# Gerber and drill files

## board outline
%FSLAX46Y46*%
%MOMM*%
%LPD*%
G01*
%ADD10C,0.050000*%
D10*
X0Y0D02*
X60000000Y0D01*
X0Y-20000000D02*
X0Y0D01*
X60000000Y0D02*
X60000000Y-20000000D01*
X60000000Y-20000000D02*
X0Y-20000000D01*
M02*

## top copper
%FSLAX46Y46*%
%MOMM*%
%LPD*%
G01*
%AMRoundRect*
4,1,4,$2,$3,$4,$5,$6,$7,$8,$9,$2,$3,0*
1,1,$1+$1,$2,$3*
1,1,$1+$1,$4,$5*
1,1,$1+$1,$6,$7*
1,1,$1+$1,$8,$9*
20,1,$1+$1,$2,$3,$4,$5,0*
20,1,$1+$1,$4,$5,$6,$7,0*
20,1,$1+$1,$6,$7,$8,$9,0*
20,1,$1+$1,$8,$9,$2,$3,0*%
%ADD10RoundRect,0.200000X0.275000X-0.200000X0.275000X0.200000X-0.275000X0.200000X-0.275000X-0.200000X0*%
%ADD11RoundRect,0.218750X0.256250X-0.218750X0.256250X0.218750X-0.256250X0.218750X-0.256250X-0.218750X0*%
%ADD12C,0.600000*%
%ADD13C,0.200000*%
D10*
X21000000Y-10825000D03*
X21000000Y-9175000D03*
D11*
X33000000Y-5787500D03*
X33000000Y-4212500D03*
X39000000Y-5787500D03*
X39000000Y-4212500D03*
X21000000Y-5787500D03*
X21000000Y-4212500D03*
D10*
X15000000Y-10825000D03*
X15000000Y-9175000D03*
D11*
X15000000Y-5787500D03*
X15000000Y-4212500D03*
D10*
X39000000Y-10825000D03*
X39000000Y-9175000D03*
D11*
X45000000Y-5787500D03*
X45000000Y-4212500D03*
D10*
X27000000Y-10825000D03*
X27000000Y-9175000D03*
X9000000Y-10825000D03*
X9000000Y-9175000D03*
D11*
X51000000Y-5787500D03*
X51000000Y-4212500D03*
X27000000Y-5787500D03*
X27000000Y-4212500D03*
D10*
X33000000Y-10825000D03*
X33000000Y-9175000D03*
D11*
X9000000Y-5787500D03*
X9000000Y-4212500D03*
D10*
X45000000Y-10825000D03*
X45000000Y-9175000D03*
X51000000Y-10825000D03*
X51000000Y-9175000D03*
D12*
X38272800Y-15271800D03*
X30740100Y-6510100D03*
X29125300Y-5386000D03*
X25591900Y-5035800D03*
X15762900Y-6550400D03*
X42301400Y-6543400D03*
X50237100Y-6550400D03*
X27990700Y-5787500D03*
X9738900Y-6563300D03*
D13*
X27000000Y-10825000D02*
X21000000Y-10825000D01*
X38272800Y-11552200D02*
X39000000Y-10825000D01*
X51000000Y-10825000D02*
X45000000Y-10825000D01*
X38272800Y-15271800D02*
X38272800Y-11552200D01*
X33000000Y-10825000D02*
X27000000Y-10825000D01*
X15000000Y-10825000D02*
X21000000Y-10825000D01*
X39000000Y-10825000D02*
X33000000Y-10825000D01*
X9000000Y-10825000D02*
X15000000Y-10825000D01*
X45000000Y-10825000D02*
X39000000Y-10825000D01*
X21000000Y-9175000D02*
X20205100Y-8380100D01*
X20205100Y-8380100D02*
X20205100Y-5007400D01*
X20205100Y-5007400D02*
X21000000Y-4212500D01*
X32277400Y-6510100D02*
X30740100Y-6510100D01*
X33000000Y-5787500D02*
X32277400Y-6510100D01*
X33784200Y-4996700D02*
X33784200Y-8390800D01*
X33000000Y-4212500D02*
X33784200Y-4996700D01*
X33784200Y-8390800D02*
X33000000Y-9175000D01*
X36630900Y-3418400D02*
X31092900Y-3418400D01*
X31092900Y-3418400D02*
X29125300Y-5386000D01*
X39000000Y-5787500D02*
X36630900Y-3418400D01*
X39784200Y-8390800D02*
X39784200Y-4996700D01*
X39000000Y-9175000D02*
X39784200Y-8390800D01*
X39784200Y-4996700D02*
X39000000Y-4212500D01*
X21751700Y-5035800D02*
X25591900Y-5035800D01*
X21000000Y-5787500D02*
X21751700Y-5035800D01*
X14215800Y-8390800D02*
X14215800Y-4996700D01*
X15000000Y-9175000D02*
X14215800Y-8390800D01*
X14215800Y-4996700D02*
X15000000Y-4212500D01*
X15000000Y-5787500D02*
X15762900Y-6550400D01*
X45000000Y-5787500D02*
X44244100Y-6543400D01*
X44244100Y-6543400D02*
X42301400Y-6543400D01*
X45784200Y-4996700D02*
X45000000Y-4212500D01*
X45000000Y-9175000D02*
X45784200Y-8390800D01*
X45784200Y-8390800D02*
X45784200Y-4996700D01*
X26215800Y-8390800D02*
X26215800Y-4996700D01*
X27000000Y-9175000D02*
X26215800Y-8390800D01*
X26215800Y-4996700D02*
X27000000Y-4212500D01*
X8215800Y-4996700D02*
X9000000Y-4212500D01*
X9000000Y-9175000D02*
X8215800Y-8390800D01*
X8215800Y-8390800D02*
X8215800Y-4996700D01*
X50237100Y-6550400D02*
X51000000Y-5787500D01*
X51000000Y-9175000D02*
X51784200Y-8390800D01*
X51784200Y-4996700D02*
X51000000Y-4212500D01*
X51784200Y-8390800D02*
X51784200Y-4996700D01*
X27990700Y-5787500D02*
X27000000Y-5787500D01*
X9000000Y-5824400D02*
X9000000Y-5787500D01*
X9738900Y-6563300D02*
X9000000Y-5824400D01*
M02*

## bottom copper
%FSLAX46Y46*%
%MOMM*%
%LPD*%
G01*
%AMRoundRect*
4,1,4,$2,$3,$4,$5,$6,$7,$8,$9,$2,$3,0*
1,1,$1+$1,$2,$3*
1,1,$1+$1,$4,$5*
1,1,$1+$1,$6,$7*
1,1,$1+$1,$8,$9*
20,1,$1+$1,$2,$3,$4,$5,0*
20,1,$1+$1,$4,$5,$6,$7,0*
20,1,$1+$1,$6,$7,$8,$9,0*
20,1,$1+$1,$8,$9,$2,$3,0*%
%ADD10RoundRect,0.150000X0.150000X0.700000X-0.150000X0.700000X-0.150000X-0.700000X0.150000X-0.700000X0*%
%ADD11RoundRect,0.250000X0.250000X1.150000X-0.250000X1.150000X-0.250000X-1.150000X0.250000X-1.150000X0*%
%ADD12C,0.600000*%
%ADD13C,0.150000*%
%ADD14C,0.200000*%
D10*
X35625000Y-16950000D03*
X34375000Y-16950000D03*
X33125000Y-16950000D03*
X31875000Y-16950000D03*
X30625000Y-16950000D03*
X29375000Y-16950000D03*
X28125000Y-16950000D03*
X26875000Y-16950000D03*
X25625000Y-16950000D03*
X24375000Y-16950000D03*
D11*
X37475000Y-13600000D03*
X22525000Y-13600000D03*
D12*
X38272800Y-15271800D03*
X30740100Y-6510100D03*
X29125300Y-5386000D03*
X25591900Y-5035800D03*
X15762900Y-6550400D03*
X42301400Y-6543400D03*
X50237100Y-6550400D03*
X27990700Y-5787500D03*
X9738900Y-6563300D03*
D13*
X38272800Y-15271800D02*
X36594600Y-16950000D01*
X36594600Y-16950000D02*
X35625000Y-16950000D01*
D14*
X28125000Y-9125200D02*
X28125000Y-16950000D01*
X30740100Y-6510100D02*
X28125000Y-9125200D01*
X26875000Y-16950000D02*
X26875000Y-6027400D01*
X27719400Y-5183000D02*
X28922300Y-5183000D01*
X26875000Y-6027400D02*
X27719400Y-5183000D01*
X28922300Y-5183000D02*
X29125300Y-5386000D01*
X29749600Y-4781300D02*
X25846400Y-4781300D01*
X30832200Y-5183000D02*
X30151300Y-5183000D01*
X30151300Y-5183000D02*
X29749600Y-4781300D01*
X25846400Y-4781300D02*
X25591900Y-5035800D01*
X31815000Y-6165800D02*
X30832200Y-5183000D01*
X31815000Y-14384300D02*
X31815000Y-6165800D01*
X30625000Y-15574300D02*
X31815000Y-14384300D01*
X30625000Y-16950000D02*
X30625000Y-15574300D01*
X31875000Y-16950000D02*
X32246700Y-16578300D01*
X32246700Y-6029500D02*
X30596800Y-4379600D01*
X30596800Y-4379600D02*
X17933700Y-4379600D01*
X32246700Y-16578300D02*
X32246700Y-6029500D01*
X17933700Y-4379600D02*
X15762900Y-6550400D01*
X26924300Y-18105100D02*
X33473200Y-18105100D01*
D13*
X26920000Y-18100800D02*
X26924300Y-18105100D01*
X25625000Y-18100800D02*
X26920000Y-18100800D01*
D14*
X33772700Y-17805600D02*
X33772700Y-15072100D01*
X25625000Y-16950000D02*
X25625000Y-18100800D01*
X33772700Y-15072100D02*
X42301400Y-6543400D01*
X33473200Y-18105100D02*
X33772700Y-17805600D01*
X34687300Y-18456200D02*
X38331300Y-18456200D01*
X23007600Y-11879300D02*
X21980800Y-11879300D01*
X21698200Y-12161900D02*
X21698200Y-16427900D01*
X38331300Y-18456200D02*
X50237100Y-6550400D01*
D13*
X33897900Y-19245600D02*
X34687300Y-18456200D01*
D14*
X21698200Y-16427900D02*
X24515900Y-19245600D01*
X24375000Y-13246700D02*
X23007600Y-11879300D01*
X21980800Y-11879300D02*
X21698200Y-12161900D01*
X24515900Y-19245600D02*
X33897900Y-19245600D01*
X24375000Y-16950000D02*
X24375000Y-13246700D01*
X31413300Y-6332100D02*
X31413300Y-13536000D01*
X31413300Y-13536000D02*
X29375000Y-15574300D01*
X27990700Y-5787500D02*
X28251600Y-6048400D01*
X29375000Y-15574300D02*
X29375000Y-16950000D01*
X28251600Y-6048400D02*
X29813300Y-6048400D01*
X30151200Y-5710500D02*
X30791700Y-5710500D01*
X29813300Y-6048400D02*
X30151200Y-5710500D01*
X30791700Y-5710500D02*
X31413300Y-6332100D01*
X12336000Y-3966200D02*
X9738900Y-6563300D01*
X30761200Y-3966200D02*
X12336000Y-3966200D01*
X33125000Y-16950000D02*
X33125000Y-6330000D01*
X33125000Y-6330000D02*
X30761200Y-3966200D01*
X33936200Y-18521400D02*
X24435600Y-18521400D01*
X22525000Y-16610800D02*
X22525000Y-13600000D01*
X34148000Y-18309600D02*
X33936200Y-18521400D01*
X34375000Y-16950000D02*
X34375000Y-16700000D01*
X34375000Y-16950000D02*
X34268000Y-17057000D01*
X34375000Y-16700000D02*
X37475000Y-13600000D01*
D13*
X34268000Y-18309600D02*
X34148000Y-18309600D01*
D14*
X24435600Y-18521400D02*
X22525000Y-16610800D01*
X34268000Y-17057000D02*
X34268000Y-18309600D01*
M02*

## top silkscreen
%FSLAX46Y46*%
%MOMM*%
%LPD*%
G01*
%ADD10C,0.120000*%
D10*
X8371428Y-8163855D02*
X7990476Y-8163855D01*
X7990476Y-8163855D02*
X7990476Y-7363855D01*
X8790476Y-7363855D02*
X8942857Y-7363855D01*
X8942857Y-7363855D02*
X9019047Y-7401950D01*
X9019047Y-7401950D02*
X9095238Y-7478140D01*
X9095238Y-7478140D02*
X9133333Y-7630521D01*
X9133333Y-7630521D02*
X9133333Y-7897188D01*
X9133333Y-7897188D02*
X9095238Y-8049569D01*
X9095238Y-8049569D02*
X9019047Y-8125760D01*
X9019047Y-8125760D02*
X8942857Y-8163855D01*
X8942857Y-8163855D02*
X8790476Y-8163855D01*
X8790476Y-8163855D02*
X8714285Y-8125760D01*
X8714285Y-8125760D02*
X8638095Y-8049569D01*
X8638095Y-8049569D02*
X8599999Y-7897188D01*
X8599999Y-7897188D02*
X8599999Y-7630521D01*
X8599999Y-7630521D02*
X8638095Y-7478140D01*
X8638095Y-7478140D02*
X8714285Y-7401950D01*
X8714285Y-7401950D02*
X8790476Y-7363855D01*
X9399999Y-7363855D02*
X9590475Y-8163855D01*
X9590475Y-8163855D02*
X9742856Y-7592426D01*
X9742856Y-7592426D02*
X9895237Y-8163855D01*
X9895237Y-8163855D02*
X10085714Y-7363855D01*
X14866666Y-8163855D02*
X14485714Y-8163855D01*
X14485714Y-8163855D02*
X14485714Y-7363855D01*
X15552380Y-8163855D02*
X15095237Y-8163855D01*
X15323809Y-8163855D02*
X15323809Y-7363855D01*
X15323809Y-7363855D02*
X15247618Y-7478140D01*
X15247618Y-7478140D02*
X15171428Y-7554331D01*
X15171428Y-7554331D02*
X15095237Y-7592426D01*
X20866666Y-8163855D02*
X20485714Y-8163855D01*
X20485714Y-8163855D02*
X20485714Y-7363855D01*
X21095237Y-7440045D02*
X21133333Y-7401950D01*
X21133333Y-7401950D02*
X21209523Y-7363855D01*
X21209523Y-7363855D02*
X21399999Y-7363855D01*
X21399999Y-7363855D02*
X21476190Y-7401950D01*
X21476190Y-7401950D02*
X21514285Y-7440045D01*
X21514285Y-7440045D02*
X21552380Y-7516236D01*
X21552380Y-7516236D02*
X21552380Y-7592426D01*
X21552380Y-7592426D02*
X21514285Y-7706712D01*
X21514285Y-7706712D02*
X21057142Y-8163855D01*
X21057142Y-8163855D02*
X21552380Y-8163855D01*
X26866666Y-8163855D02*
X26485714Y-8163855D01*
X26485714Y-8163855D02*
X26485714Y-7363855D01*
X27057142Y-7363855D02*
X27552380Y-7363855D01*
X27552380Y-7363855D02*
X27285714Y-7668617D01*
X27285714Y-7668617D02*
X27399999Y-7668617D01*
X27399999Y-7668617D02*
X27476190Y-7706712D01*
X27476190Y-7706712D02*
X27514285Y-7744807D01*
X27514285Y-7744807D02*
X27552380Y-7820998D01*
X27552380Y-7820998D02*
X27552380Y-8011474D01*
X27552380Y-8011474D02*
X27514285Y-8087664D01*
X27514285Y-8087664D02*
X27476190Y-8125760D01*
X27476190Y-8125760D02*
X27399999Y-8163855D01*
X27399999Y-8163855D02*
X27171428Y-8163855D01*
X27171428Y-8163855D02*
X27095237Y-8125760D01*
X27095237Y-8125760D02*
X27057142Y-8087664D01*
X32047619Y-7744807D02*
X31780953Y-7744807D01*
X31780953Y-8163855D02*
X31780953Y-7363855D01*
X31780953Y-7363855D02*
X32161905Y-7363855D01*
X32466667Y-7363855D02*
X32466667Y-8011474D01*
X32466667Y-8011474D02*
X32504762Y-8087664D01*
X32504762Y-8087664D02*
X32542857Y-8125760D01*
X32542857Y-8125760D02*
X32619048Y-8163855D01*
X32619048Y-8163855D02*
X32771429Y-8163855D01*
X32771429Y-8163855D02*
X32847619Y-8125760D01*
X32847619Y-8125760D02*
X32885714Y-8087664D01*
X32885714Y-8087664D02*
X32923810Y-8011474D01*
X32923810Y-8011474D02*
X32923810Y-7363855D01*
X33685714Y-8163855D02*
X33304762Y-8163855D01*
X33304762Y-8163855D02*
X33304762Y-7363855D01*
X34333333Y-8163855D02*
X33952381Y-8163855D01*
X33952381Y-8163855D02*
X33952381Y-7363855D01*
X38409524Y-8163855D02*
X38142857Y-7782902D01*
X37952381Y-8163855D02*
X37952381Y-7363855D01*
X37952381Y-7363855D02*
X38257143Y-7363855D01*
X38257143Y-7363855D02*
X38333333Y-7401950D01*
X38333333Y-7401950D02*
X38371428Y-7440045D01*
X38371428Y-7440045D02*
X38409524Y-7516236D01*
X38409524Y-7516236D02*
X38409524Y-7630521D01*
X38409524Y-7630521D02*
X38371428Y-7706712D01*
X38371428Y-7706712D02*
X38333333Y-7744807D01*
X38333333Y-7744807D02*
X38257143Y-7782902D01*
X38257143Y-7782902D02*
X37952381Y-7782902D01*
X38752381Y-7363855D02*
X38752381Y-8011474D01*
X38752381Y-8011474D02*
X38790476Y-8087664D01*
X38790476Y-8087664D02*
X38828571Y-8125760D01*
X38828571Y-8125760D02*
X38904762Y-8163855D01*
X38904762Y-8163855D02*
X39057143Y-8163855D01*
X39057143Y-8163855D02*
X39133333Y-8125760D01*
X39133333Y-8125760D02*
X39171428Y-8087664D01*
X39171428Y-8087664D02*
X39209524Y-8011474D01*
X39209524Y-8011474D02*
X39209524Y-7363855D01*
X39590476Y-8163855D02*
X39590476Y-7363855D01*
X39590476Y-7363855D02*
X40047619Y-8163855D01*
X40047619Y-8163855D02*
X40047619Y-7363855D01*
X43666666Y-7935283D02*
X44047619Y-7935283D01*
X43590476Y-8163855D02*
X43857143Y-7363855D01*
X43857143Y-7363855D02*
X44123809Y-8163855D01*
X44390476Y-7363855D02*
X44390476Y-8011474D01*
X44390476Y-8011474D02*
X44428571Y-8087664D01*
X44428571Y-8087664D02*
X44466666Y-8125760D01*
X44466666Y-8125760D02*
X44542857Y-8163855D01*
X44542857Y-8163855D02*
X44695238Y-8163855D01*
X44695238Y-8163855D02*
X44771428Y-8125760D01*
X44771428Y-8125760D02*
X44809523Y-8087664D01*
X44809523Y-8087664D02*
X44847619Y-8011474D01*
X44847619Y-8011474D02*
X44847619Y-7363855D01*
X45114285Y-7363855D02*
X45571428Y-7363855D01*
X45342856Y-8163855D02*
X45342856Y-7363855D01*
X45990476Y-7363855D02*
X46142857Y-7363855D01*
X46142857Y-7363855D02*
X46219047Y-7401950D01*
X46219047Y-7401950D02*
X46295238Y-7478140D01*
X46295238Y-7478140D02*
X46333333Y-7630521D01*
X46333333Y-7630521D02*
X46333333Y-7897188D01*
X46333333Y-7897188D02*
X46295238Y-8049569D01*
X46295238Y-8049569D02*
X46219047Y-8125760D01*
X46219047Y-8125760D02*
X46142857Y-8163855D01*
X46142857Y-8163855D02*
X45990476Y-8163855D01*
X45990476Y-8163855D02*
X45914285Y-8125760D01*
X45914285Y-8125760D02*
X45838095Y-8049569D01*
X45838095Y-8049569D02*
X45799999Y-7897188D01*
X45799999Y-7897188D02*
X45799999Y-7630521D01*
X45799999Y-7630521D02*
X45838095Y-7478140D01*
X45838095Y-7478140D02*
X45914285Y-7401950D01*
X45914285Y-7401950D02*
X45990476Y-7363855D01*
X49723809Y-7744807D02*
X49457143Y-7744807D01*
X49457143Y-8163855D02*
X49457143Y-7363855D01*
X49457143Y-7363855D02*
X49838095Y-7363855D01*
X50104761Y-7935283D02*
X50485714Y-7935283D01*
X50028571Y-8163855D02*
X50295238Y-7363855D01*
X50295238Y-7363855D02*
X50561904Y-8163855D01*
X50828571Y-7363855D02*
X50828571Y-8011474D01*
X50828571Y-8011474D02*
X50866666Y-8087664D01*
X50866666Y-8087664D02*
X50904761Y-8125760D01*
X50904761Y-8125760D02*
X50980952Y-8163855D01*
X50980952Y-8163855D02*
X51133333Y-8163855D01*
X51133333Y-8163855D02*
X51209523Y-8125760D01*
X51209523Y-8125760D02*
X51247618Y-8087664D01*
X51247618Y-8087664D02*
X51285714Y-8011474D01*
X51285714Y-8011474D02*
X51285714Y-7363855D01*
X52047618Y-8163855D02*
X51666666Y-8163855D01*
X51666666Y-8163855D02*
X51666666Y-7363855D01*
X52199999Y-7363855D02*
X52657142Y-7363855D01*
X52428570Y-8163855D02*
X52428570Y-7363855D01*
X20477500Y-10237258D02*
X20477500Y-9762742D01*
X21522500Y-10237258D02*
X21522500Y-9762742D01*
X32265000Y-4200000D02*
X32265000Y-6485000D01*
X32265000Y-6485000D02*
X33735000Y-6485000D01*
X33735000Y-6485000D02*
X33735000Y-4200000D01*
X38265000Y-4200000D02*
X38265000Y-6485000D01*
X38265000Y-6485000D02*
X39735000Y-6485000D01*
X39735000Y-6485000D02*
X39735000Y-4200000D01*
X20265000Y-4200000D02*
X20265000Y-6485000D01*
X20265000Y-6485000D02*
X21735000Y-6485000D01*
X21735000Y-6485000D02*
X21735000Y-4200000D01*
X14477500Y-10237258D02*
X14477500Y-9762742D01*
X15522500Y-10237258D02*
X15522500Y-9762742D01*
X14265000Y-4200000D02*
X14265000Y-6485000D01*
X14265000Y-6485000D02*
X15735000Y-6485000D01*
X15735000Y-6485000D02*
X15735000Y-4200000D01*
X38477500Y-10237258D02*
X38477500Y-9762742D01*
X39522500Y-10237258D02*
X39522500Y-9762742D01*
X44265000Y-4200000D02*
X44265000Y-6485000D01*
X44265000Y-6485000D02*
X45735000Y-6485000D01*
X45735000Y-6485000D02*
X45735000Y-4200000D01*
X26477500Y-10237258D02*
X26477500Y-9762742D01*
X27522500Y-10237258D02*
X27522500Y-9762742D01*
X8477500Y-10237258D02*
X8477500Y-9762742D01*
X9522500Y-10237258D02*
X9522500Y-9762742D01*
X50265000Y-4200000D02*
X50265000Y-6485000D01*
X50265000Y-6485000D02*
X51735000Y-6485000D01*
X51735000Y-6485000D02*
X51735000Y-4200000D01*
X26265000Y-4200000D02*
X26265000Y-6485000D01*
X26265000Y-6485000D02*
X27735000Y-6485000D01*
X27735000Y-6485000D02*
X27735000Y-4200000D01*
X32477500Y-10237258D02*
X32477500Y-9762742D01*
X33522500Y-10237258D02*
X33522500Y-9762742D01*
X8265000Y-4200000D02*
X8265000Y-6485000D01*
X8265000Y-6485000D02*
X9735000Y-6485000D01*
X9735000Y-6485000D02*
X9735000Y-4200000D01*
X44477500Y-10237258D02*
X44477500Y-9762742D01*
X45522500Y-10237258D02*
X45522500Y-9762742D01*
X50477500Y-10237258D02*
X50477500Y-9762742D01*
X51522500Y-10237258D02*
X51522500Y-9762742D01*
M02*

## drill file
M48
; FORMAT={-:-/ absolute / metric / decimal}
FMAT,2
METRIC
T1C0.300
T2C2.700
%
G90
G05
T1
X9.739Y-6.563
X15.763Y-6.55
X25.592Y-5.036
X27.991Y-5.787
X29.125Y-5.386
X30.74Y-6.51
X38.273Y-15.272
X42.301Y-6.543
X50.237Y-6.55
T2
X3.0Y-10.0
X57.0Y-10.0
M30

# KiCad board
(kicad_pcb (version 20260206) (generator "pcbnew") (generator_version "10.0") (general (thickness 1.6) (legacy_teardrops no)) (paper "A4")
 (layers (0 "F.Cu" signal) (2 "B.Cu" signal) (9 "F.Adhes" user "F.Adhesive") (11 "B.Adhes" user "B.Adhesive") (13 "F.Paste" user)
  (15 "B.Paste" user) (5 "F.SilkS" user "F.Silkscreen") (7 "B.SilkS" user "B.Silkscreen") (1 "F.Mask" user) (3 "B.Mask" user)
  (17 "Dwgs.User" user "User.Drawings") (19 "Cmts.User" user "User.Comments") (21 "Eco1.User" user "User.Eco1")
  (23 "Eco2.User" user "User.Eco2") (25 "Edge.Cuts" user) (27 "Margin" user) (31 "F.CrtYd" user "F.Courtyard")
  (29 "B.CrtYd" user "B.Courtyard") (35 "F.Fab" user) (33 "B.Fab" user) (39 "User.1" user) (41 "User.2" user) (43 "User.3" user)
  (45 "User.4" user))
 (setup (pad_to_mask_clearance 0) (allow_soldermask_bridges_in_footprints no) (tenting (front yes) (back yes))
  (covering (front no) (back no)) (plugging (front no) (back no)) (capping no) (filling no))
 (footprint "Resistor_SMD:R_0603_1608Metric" (layer "F.Cu") (at 21 10 90)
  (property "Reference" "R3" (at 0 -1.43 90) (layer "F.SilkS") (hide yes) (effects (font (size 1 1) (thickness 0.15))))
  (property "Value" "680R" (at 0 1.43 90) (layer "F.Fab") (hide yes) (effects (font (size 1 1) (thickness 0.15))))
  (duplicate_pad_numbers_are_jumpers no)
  (fp_line (start -0.237258 -0.5225) (end 0.237258 -0.5225) (stroke (width 0.12) (type solid)) (layer "F.SilkS"))
  (fp_line (start -0.237258 0.5225) (end 0.237258 0.5225) (stroke (width 0.12) (type solid)) (layer "F.SilkS"))
  (pad "1" smd roundrect (at -0.825 0 90) (size 0.8 0.95) (layers "F.Cu" "F.Mask" "F.Paste") (roundrect_rratio 0.25) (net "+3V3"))
  (pad "2" smd roundrect (at 0.825 0 90) (size 0.8 0.95) (layers "F.Cu" "F.Mask" "F.Paste") (roundrect_rratio 0.25) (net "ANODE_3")))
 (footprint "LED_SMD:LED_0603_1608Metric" (layer "F.Cu") (at 33 5 90)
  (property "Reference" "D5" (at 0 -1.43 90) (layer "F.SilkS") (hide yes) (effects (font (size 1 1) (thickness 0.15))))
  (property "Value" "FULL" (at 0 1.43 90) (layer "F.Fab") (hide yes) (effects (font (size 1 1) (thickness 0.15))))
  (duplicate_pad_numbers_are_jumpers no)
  (fp_line (start 0.8 -0.735) (end -1.485 -0.735) (stroke (width 0.12) (type solid)) (layer "F.SilkS"))
  (fp_line (start -1.485 -0.735) (end -1.485 0.735) (stroke (width 0.12) (type solid)) (layer "F.SilkS"))
  (fp_line (start -1.485 0.735) (end 0.8 0.735) (stroke (width 0.12) (type solid)) (layer "F.SilkS"))
  (pad "1" smd roundrect (at -0.7875 0 90) (size 0.875 0.95) (layers "F.Cu" "F.Mask" "F.Paste") (roundrect_rratio 0.25) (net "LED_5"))
  (pad "2" smd roundrect (at 0.7875 0 90) (size 0.875 0.95) (layers "F.Cu" "F.Mask" "F.Paste") (roundrect_rratio 0.25) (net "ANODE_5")))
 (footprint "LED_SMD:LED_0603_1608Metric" (layer "F.Cu") (at 39 5 90)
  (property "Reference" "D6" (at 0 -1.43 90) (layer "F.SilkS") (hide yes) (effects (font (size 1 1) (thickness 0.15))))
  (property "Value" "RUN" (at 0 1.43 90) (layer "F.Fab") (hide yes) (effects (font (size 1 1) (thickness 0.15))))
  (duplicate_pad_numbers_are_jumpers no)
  (fp_line (start 0.8 -0.735) (end -1.485 -0.735) (stroke (width 0.12) (type solid)) (layer "F.SilkS"))
  (fp_line (start -1.485 -0.735) (end -1.485 0.735) (stroke (width 0.12) (type solid)) (layer "F.SilkS"))
  (fp_line (start -1.485 0.735) (end 0.8 0.735) (stroke (width 0.12) (type solid)) (layer "F.SilkS"))
  (pad "1" smd roundrect (at -0.7875 0 90) (size 0.875 0.95) (layers "F.Cu" "F.Mask" "F.Paste") (roundrect_rratio 0.25) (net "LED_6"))
  (pad "2" smd roundrect (at 0.7875 0 90) (size 0.875 0.95) (layers "F.Cu" "F.Mask" "F.Paste") (roundrect_rratio 0.25) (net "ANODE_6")))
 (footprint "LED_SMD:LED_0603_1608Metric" (layer "F.Cu") (at 21 5 90)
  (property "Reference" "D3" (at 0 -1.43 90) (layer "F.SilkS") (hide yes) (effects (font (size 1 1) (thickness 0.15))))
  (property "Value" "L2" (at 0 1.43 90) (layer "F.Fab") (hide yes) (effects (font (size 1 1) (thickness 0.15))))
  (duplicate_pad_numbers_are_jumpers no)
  (fp_line (start 0.8 -0.735) (end -1.485 -0.735) (stroke (width 0.12) (type solid)) (layer "F.SilkS"))
  (fp_line (start -1.485 -0.735) (end -1.485 0.735) (stroke (width 0.12) (type solid)) (layer "F.SilkS"))
  (fp_line (start -1.485 0.735) (end 0.8 0.735) (stroke (width 0.12) (type solid)) (layer "F.SilkS"))
  (pad "1" smd roundrect (at -0.7875 0 90) (size 0.875 0.95) (layers "F.Cu" "F.Mask" "F.Paste") (roundrect_rratio 0.25) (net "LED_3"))
  (pad "2" smd roundrect (at 0.7875 0 90) (size 0.875 0.95) (layers "F.Cu" "F.Mask" "F.Paste") (roundrect_rratio 0.25) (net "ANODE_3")))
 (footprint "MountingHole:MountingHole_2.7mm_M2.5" (layer "F.Cu") (at 3 10)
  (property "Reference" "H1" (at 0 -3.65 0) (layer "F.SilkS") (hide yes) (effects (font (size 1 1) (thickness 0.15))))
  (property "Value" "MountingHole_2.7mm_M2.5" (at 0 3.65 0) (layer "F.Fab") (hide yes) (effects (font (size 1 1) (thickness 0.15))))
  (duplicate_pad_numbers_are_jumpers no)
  (pad "" np_thru_hole circle (at 0 0) (size 2.7 2.7) (drill 2.7) (layers "*.Cu" "*.Mask")))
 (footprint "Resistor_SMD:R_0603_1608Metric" (layer "F.Cu") (at 15 10 90)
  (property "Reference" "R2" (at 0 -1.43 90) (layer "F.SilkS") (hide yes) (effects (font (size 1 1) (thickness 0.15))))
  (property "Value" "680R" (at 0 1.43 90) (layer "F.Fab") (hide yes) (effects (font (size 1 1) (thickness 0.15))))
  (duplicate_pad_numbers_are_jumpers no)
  (fp_line (start -0.237258 -0.5225) (end 0.237258 -0.5225) (stroke (width 0.12) (type solid)) (layer "F.SilkS"))
  (fp_line (start -0.237258 0.5225) (end 0.237258 0.5225) (stroke (width 0.12) (type solid)) (layer "F.SilkS"))
  (pad "1" smd roundrect (at -0.825 0 90) (size 0.8 0.95) (layers "F.Cu" "F.Mask" "F.Paste") (roundrect_rratio 0.25) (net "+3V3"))
  (pad "2" smd roundrect (at 0.825 0 90) (size 0.8 0.95) (layers "F.Cu" "F.Mask" "F.Paste") (roundrect_rratio 0.25) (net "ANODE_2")))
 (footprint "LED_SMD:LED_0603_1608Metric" (layer "F.Cu") (at 15 5 90)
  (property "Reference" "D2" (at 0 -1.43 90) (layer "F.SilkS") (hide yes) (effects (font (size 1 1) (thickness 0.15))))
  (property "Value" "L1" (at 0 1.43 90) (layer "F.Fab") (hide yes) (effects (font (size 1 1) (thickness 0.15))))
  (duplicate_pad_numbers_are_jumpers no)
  (fp_line (start 0.8 -0.735) (end -1.485 -0.735) (stroke (width 0.12) (type solid)) (layer "F.SilkS"))
  (fp_line (start -1.485 -0.735) (end -1.485 0.735) (stroke (width 0.12) (type solid)) (layer "F.SilkS"))
  (fp_line (start -1.485 0.735) (end 0.8 0.735) (stroke (width 0.12) (type solid)) (layer "F.SilkS"))
  (pad "1" smd roundrect (at -0.7875 0 90) (size 0.875 0.95) (layers "F.Cu" "F.Mask" "F.Paste") (roundrect_rratio 0.25) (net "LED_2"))
  (pad "2" smd roundrect (at 0.7875 0 90) (size 0.875 0.95) (layers "F.Cu" "F.Mask" "F.Paste") (roundrect_rratio 0.25) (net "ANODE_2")))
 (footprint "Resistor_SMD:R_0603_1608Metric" (layer "F.Cu") (at 39 10 90)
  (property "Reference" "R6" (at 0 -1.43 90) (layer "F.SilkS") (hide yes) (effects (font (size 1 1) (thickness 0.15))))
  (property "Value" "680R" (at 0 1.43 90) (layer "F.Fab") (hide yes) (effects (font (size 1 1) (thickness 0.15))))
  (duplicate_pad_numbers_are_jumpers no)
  (fp_line (start -0.237258 -0.5225) (end 0.237258 -0.5225) (stroke (width 0.12) (type solid)) (layer "F.SilkS"))
  (fp_line (start -0.237258 0.5225) (end 0.237258 0.5225) (stroke (width 0.12) (type solid)) (layer "F.SilkS"))
  (pad "1" smd roundrect (at -0.825 0 90) (size 0.8 0.95) (layers "F.Cu" "F.Mask" "F.Paste") (roundrect_rratio 0.25) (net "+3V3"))
  (pad "2" smd roundrect (at 0.825 0 90) (size 0.8 0.95) (layers "F.Cu" "F.Mask" "F.Paste") (roundrect_rratio 0.25) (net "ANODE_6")))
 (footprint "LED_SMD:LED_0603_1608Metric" (layer "F.Cu") (at 45 5 90)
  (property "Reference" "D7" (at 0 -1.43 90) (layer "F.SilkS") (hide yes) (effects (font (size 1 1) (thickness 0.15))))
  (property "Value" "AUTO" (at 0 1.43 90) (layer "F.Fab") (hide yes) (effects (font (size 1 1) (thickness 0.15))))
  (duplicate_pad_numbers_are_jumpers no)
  (fp_line (start 0.8 -0.735) (end -1.485 -0.735) (stroke (width 0.12) (type solid)) (layer "F.SilkS"))
  (fp_line (start -1.485 -0.735) (end -1.485 0.735) (stroke (width 0.12) (type solid)) (layer "F.SilkS"))
  (fp_line (start -1.485 0.735) (end 0.8 0.735) (stroke (width 0.12) (type solid)) (layer "F.SilkS"))
  (pad "1" smd roundrect (at -0.7875 0 90) (size 0.875 0.95) (layers "F.Cu" "F.Mask" "F.Paste") (roundrect_rratio 0.25) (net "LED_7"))
  (pad "2" smd roundrect (at 0.7875 0 90) (size 0.875 0.95) (layers "F.Cu" "F.Mask" "F.Paste") (roundrect_rratio 0.25) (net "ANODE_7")))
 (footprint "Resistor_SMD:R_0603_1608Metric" (layer "F.Cu") (at 27 10 90)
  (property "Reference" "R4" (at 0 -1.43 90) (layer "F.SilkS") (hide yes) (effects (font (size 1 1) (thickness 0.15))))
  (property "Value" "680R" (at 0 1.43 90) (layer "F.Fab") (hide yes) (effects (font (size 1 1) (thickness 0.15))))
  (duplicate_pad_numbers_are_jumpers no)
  (fp_line (start -0.237258 -0.5225) (end 0.237258 -0.5225) (stroke (width 0.12) (type solid)) (layer "F.SilkS"))
  (fp_line (start -0.237258 0.5225) (end 0.237258 0.5225) (stroke (width 0.12) (type solid)) (layer "F.SilkS"))
  (pad "1" smd roundrect (at -0.825 0 90) (size 0.8 0.95) (layers "F.Cu" "F.Mask" "F.Paste") (roundrect_rratio 0.25) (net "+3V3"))
  (pad "2" smd roundrect (at 0.825 0 90) (size 0.8 0.95) (layers "F.Cu" "F.Mask" "F.Paste") (roundrect_rratio 0.25) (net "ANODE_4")))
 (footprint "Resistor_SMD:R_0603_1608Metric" (layer "F.Cu") (at 9 10 90)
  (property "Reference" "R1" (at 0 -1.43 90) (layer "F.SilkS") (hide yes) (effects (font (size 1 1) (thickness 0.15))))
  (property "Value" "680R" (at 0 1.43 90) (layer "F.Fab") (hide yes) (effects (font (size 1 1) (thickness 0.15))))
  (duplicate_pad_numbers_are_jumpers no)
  (fp_line (start -0.237258 -0.5225) (end 0.237258 -0.5225) (stroke (width 0.12) (type solid)) (layer "F.SilkS"))
  (fp_line (start -0.237258 0.5225) (end 0.237258 0.5225) (stroke (width 0.12) (type solid)) (layer "F.SilkS"))
  (pad "1" smd roundrect (at -0.825 0 90) (size 0.8 0.95) (layers "F.Cu" "F.Mask" "F.Paste") (roundrect_rratio 0.25) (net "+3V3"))
  (pad "2" smd roundrect (at 0.825 0 90) (size 0.8 0.95) (layers "F.Cu" "F.Mask" "F.Paste") (roundrect_rratio 0.25) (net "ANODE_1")))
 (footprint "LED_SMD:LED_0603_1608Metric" (layer "F.Cu") (at 51 5 90)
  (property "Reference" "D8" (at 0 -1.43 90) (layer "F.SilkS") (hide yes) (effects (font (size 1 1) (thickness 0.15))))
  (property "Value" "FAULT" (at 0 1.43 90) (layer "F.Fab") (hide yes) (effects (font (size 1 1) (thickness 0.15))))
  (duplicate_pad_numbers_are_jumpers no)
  (fp_line (start 0.8 -0.735) (end -1.485 -0.735) (stroke (width 0.12) (type solid)) (layer "F.SilkS"))
  (fp_line (start -1.485 -0.735) (end -1.485 0.735) (stroke (width 0.12) (type solid)) (layer "F.SilkS"))
  (fp_line (start -1.485 0.735) (end 0.8 0.735) (stroke (width 0.12) (type solid)) (layer "F.SilkS"))
  (pad "1" smd roundrect (at -0.7875 0 90) (size 0.875 0.95) (layers "F.Cu" "F.Mask" "F.Paste") (roundrect_rratio 0.25) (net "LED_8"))
  (pad "2" smd roundrect (at 0.7875 0 90) (size 0.875 0.95) (layers "F.Cu" "F.Mask" "F.Paste") (roundrect_rratio 0.25) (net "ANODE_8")))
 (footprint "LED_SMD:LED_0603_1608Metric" (layer "F.Cu") (at 27 5 90)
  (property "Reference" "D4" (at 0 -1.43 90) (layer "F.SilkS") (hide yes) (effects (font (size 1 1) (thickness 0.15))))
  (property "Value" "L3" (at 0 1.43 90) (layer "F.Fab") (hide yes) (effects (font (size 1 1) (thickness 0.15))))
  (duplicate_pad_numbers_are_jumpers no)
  (fp_line (start 0.8 -0.735) (end -1.485 -0.735) (stroke (width 0.12) (type solid)) (layer "F.SilkS"))
  (fp_line (start -1.485 -0.735) (end -1.485 0.735) (stroke (width 0.12) (type solid)) (layer "F.SilkS"))
  (fp_line (start -1.485 0.735) (end 0.8 0.735) (stroke (width 0.12) (type solid)) (layer "F.SilkS"))
  (pad "1" smd roundrect (at -0.7875 0 90) (size 0.875 0.95) (layers "F.Cu" "F.Mask" "F.Paste") (roundrect_rratio 0.25) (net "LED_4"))
  (pad "2" smd roundrect (at 0.7875 0 90) (size 0.875 0.95) (layers "F.Cu" "F.Mask" "F.Paste") (roundrect_rratio 0.25) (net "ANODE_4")))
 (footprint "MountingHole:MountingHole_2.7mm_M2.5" (layer "F.Cu") (at 57 10)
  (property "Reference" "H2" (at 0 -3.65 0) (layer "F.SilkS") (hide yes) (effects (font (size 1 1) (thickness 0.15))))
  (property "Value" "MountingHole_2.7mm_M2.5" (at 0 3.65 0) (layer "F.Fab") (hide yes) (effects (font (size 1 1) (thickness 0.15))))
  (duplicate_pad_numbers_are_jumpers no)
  (pad "" np_thru_hole circle (at 0 0) (size 2.7 2.7) (drill 2.7) (layers "*.Cu" "*.Mask")))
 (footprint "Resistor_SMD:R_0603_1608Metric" (layer "F.Cu") (at 33 10 90)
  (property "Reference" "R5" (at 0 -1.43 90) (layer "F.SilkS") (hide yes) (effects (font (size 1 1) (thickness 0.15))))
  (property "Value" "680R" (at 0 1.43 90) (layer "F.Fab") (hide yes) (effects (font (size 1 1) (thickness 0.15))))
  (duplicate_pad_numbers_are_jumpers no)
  (fp_line (start -0.237258 -0.5225) (end 0.237258 -0.5225) (stroke (width 0.12) (type solid)) (layer "F.SilkS"))
  (fp_line (start -0.237258 0.5225) (end 0.237258 0.5225) (stroke (width 0.12) (type solid)) (layer "F.SilkS"))
  (pad "1" smd roundrect (at -0.825 0 90) (size 0.8 0.95) (layers "F.Cu" "F.Mask" "F.Paste") (roundrect_rratio 0.25) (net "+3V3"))
  (pad "2" smd roundrect (at 0.825 0 90) (size 0.8 0.95) (layers "F.Cu" "F.Mask" "F.Paste") (roundrect_rratio 0.25) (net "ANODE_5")))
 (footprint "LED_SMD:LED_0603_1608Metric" (layer "F.Cu") (at 9 5 90)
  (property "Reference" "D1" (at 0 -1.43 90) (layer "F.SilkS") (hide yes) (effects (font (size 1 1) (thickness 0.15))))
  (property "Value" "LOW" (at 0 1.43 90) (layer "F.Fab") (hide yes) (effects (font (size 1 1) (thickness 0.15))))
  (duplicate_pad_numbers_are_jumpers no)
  (fp_line (start 0.8 -0.735) (end -1.485 -0.735) (stroke (width 0.12) (type solid)) (layer "F.SilkS"))
  (fp_line (start -1.485 -0.735) (end -1.485 0.735) (stroke (width 0.12) (type solid)) (layer "F.SilkS"))
  (fp_line (start -1.485 0.735) (end 0.8 0.735) (stroke (width 0.12) (type solid)) (layer "F.SilkS"))
  (pad "1" smd roundrect (at -0.7875 0 90) (size 0.875 0.95) (layers "F.Cu" "F.Mask" "F.Paste") (roundrect_rratio 0.25) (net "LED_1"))
  (pad "2" smd roundrect (at 0.7875 0 90) (size 0.875 0.95) (layers "F.Cu" "F.Mask" "F.Paste") (roundrect_rratio 0.25) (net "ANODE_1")))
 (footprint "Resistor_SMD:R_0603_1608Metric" (layer "F.Cu") (at 45 10 90)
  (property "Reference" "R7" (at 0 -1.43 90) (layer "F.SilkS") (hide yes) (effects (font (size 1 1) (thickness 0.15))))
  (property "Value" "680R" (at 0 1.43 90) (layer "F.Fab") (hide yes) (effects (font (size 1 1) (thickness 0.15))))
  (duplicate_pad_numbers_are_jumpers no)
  (fp_line (start -0.237258 -0.5225) (end 0.237258 -0.5225) (stroke (width 0.12) (type solid)) (layer "F.SilkS"))
  (fp_line (start -0.237258 0.5225) (end 0.237258 0.5225) (stroke (width 0.12) (type solid)) (layer "F.SilkS"))
  (pad "1" smd roundrect (at -0.825 0 90) (size 0.8 0.95) (layers "F.Cu" "F.Mask" "F.Paste") (roundrect_rratio 0.25) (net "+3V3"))
  (pad "2" smd roundrect (at 0.825 0 90) (size 0.8 0.95) (layers "F.Cu" "F.Mask" "F.Paste") (roundrect_rratio 0.25) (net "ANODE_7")))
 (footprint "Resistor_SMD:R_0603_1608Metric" (layer "F.Cu") (at 51 10 90)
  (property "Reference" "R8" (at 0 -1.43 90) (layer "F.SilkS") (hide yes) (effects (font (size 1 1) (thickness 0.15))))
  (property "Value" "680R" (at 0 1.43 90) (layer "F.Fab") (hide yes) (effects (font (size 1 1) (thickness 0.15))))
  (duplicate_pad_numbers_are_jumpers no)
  (fp_line (start -0.237258 -0.5225) (end 0.237258 -0.5225) (stroke (width 0.12) (type solid)) (layer "F.SilkS"))
  (fp_line (start -0.237258 0.5225) (end 0.237258 0.5225) (stroke (width 0.12) (type solid)) (layer "F.SilkS"))
  (pad "1" smd roundrect (at -0.825 0 90) (size 0.8 0.95) (layers "F.Cu" "F.Mask" "F.Paste") (roundrect_rratio 0.25) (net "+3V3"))
  (pad "2" smd roundrect (at 0.825 0 90) (size 0.8 0.95) (layers "F.Cu" "F.Mask" "F.Paste") (roundrect_rratio 0.25) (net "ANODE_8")))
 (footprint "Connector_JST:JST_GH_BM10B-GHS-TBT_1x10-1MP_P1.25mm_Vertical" (layer "B.Cu") (at 30 15 180)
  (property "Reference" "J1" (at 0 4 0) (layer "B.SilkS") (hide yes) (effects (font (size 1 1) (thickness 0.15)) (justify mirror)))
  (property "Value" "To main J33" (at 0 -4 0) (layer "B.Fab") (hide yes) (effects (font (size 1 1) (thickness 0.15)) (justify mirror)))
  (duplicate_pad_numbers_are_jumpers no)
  (pad "1" smd roundrect (at -5.625 -1.95 180) (size 0.6 1.7) (layers "B.Cu" "B.Mask" "B.Paste") (roundrect_rratio 0.25) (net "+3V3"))
  (pad "2" smd roundrect (at -4.375 -1.95 180) (size 0.6 1.7) (layers "B.Cu" "B.Mask" "B.Paste") (roundrect_rratio 0.25) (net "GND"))
  (pad "3" smd roundrect (at -3.125 -1.95 180) (size 0.6 1.7) (layers "B.Cu" "B.Mask" "B.Paste") (roundrect_rratio 0.25) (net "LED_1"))
  (pad "4" smd roundrect (at -1.875 -1.95 180) (size 0.6 1.7) (layers "B.Cu" "B.Mask" "B.Paste") (roundrect_rratio 0.25) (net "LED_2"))
  (pad "5" smd roundrect (at -0.625 -1.95 180) (size 0.6 1.7) (layers "B.Cu" "B.Mask" "B.Paste") (roundrect_rratio 0.25) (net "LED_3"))
  (pad "6" smd roundrect (at 0.625 -1.95 180) (size 0.6 1.7) (layers "B.Cu" "B.Mask" "B.Paste") (roundrect_rratio 0.25) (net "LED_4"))
  (pad "7" smd roundrect (at 1.875 -1.95 180) (size 0.6 1.7) (layers "B.Cu" "B.Mask" "B.Paste") (roundrect_rratio 0.25) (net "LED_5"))
  (pad "8" smd roundrect (at 3.125 -1.95 180) (size 0.6 1.7) (layers "B.Cu" "B.Mask" "B.Paste") (roundrect_rratio 0.25) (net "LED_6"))
  (pad "9" smd roundrect (at 4.375 -1.95 180) (size 0.6 1.7) (layers "B.Cu" "B.Mask" "B.Paste") (roundrect_rratio 0.25) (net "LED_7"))
  (pad "10" smd roundrect (at 5.625 -1.95 180) (size 0.6 1.7) (layers "B.Cu" "B.Mask" "B.Paste") (roundrect_rratio 0.25) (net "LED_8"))
  (pad "MP" smd roundrect (at -7.475 1.4 180) (size 1 2.8) (layers "B.Cu" "B.Mask" "B.Paste") (roundrect_rratio 0.25) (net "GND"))
  (pad "MP" smd roundrect (at 7.475 1.4 180) (size 1 2.8) (layers "B.Cu" "B.Mask" "B.Paste") (roundrect_rratio 0.25) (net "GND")))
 (gr_line (start 0 0) (end 60 0) (stroke (width 0.05) (type default)) (layer "Edge.Cuts"))
 (gr_line (start 0 20) (end 0 0) (stroke (width 0.05) (type default)) (layer "Edge.Cuts"))
 (gr_line (start 60 0) (end 60 20) (stroke (width 0.05) (type default)) (layer "Edge.Cuts"))
 (gr_line (start 60 20) (end 0 20) (stroke (width 0.05) (type default)) (layer "Edge.Cuts"))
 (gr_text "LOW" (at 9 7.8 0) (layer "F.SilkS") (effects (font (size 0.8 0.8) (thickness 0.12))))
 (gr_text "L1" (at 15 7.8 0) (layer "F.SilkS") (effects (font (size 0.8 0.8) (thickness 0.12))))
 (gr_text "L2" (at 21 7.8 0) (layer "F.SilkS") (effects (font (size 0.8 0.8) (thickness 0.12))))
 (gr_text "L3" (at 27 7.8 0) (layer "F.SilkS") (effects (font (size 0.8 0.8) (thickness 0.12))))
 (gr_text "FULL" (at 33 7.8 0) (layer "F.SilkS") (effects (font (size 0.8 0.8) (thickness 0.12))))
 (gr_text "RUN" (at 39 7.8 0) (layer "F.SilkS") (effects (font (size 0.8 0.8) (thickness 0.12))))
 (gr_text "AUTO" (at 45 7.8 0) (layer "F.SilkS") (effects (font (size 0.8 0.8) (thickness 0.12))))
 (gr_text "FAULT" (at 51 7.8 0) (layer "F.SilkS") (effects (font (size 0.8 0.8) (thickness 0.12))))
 (segment (start 27 10.825) (end 21 10.825) (width 0.2) (layer "F.Cu") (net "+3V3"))
 (segment (start 38.2728 11.5522) (end 39 10.825) (width 0.2) (layer "F.Cu") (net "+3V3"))
 (segment (start 51 10.825) (end 45 10.825) (width 0.2) (layer "F.Cu") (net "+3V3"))
 (segment (start 38.2728 15.2718) (end 38.2728 11.5522) (width 0.2) (layer "F.Cu") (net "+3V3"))
 (segment (start 33 10.825) (end 27 10.825) (width 0.2) (layer "F.Cu") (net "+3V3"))
 (segment (start 15 10.825) (end 21 10.825) (width 0.2) (layer "F.Cu") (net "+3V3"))
 (segment (start 39 10.825) (end 33 10.825) (width 0.2) (layer "F.Cu") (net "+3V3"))
 (segment (start 9 10.825) (end 15 10.825) (width 0.2) (layer "F.Cu") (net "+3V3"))
 (segment (start 45 10.825) (end 39 10.825) (width 0.2) (layer "F.Cu") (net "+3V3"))
 (via (at 38.2728 15.2718) (size 0.6) (drill 0.3) (layers "F.Cu" "B.Cu") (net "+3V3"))
 (segment (start 38.2728 15.2718) (end 36.5946 16.95) (width 0.15) (layer "B.Cu") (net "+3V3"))
 (segment (start 36.5946 16.95) (end 35.625 16.95) (width 0.15) (layer "B.Cu") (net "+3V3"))
 (segment (start 21 9.175) (end 20.2051 8.3801) (width 0.2) (layer "F.Cu") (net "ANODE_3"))
 (segment (start 20.2051 8.3801) (end 20.2051 5.0074) (width 0.2) (layer "F.Cu") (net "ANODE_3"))
 (segment (start 20.2051 5.0074) (end 21 4.2125) (width 0.2) (layer "F.Cu") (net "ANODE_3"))
 (segment (start 32.2774 6.5101) (end 30.7401 6.5101) (width 0.2) (layer "F.Cu") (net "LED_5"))
 (segment (start 33 5.7875) (end 32.2774 6.5101) (width 0.2) (layer "F.Cu") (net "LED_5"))
 (via (at 30.7401 6.5101) (size 0.6) (drill 0.3) (layers "F.Cu" "B.Cu") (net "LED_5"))
 (segment (start 28.125 9.1252) (end 28.125 16.95) (width 0.2) (layer "B.Cu") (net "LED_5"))
 (segment (start 30.7401 6.5101) (end 28.125 9.1252) (width 0.2) (layer "B.Cu") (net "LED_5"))
 (segment (start 33.7842 4.9967) (end 33.7842 8.3908) (width 0.2) (layer "F.Cu") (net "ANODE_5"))
 (segment (start 33 4.2125) (end 33.7842 4.9967) (width 0.2) (layer "F.Cu") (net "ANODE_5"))
 (segment (start 33.7842 8.3908) (end 33 9.175) (width 0.2) (layer "F.Cu") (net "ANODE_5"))
 (segment (start 36.6309 3.4184) (end 31.0929 3.4184) (width 0.2) (layer "F.Cu") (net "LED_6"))
 (segment (start 31.0929 3.4184) (end 29.1253 5.386) (width 0.2) (layer "F.Cu") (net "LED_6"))
 (segment (start 39 5.7875) (end 36.6309 3.4184) (width 0.2) (layer "F.Cu") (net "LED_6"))
 (via (at 29.1253 5.386) (size 0.6) (drill 0.3) (layers "F.Cu" "B.Cu") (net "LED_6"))
 (segment (start 26.875 16.95) (end 26.875 6.0274) (width 0.2) (layer "B.Cu") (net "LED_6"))
 (segment (start 27.7194 5.183) (end 28.9223 5.183) (width 0.2) (layer "B.Cu") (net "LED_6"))
 (segment (start 26.875 6.0274) (end 27.7194 5.183) (width 0.2) (layer "B.Cu") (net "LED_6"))
 (segment (start 28.9223 5.183) (end 29.1253 5.386) (width 0.2) (layer "B.Cu") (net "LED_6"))
 (segment (start 39.7842 8.3908) (end 39.7842 4.9967) (width 0.2) (layer "F.Cu") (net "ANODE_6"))
 (segment (start 39 9.175) (end 39.7842 8.3908) (width 0.2) (layer "F.Cu") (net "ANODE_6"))
 (segment (start 39.7842 4.9967) (end 39 4.2125) (width 0.2) (layer "F.Cu") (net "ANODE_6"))
 (segment (start 21.7517 5.0358) (end 25.5919 5.0358) (width 0.2) (layer "F.Cu") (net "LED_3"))
 (segment (start 21 5.7875) (end 21.7517 5.0358) (width 0.2) (layer "F.Cu") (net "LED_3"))
 (via (at 25.5919 5.0358) (size 0.6) (drill 0.3) (layers "F.Cu" "B.Cu") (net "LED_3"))
 (segment (start 29.7496 4.7813) (end 25.8464 4.7813) (width 0.2) (layer "B.Cu") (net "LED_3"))
 (segment (start 30.8322 5.183) (end 30.1513 5.183) (width 0.2) (layer "B.Cu") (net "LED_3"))
 (segment (start 30.1513 5.183) (end 29.7496 4.7813) (width 0.2) (layer "B.Cu") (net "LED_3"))
 (segment (start 25.8464 4.7813) (end 25.5919 5.0358) (width 0.2) (layer "B.Cu") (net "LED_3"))
 (segment (start 31.815 6.1658) (end 30.8322 5.183) (width 0.2) (layer "B.Cu") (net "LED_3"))
 (segment (start 31.815 14.3843) (end 31.815 6.1658) (width 0.2) (layer "B.Cu") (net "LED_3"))
 (segment (start 30.625 15.5743) (end 31.815 14.3843) (width 0.2) (layer "B.Cu") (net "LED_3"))
 (segment (start 30.625 16.95) (end 30.625 15.5743) (width 0.2) (layer "B.Cu") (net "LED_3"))
 (segment (start 14.2158 8.3908) (end 14.2158 4.9967) (width 0.2) (layer "F.Cu") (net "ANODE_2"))
 (segment (start 15 9.175) (end 14.2158 8.3908) (width 0.2) (layer "F.Cu") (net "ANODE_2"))
 (segment (start 14.2158 4.9967) (end 15 4.2125) (width 0.2) (layer "F.Cu") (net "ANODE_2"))
 (segment (start 15 5.7875) (end 15.7629 6.5504) (width 0.2) (layer "F.Cu") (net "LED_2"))
 (via (at 15.7629 6.5504) (size 0.6) (drill 0.3) (layers "F.Cu" "B.Cu") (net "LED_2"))
 (segment (start 31.875 16.95) (end 32.2467 16.5783) (width 0.2) (layer "B.Cu") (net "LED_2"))
 (segment (start 32.2467 6.0295) (end 30.5968 4.3796) (width 0.2) (layer "B.Cu") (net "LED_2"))
 (segment (start 30.5968 4.3796) (end 17.9337 4.3796) (width 0.2) (layer "B.Cu") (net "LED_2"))
 (segment (start 32.2467 16.5783) (end 32.2467 6.0295) (width 0.2) (layer "B.Cu") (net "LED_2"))
 (segment (start 17.9337 4.3796) (end 15.7629 6.5504) (width 0.2) (layer "B.Cu") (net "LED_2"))
 (segment (start 45 5.7875) (end 44.2441 6.5434) (width 0.2) (layer "F.Cu") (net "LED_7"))
 (segment (start 44.2441 6.5434) (end 42.3014 6.5434) (width 0.2) (layer "F.Cu") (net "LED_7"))
 (via (at 42.3014 6.5434) (size 0.6) (drill 0.3) (layers "F.Cu" "B.Cu") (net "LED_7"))
 (segment (start 26.9243 18.1051) (end 33.4732 18.1051) (width 0.2) (layer "B.Cu") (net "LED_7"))
 (segment (start 26.92 18.1008) (end 26.9243 18.1051) (width 0.15) (layer "B.Cu") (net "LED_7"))
 (segment (start 25.625 18.1008) (end 26.92 18.1008) (width 0.15) (layer "B.Cu") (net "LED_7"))
 (segment (start 33.7727 17.8056) (end 33.7727 15.0721) (width 0.2) (layer "B.Cu") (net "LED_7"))
 (segment (start 25.625 16.95) (end 25.625 18.1008) (width 0.2) (layer "B.Cu") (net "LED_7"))
 (segment (start 33.7727 15.0721) (end 42.3014 6.5434) (width 0.2) (layer "B.Cu") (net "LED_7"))
 (segment (start 33.4732 18.1051) (end 33.7727 17.8056) (width 0.2) (layer "B.Cu") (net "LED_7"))
 (segment (start 45.7842 4.9967) (end 45 4.2125) (width 0.2) (layer "F.Cu") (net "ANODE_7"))
 (segment (start 45 9.175) (end 45.7842 8.3908) (width 0.2) (layer "F.Cu") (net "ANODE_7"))
 (segment (start 45.7842 8.3908) (end 45.7842 4.9967) (width 0.2) (layer "F.Cu") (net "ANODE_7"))
 (segment (start 26.2158 8.3908) (end 26.2158 4.9967) (width 0.2) (layer "F.Cu") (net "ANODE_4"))
 (segment (start 27 9.175) (end 26.2158 8.3908) (width 0.2) (layer "F.Cu") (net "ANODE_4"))
 (segment (start 26.2158 4.9967) (end 27 4.2125) (width 0.2) (layer "F.Cu") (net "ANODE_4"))
 (segment (start 8.2158 4.9967) (end 9 4.2125) (width 0.2) (layer "F.Cu") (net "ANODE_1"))
 (segment (start 9 9.175) (end 8.2158 8.3908) (width 0.2) (layer "F.Cu") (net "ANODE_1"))
 (segment (start 8.2158 8.3908) (end 8.2158 4.9967) (width 0.2) (layer "F.Cu") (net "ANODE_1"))
 (segment (start 50.2371 6.5504) (end 51 5.7875) (width 0.2) (layer "F.Cu") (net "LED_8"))
 (via (at 50.2371 6.5504) (size 0.6) (drill 0.3) (layers "F.Cu" "B.Cu") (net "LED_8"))
 (segment (start 34.6873 18.4562) (end 38.3313 18.4562) (width 0.2) (layer "B.Cu") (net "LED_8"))
 (segment (start 23.0076 11.8793) (end 21.9808 11.8793) (width 0.2) (layer "B.Cu") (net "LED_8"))
 (segment (start 21.6982 12.1619) (end 21.6982 16.4279) (width 0.2) (layer "B.Cu") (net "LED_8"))
 (segment (start 38.3313 18.4562) (end 50.2371 6.5504) (width 0.2) (layer "B.Cu") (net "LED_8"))
 (segment (start 33.8979 19.2456) (end 34.6873 18.4562) (width 0.15) (layer "B.Cu") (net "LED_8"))
 (segment (start 21.6982 16.4279) (end 24.5159 19.2456) (width 0.2) (layer "B.Cu") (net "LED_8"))
 (segment (start 24.375 13.2467) (end 23.0076 11.8793) (width 0.2) (layer "B.Cu") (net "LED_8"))
 (segment (start 21.9808 11.8793) (end 21.6982 12.1619) (width 0.2) (layer "B.Cu") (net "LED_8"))
 (segment (start 24.5159 19.2456) (end 33.8979 19.2456) (width 0.2) (layer "B.Cu") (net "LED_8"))
 (segment (start 24.375 16.95) (end 24.375 13.2467) (width 0.2) (layer "B.Cu") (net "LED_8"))
 (segment (start 51 9.175) (end 51.7842 8.3908) (width 0.2) (layer "F.Cu") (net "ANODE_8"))
 (segment (start 51.7842 4.9967) (end 51 4.2125) (width 0.2) (layer "F.Cu") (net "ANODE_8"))
 (segment (start 51.7842 8.3908) (end 51.7842 4.9967) (width 0.2) (layer "F.Cu") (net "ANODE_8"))
 (segment (start 27.9907 5.7875) (end 27 5.7875) (width 0.2) (layer "F.Cu") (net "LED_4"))
 (via (at 27.9907 5.7875) (size 0.6) (drill 0.3) (layers "F.Cu" "B.Cu") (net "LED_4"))
 (segment (start 31.4133 6.3321) (end 31.4133 13.536) (width 0.2) (layer "B.Cu") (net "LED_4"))
 (segment (start 31.4133 13.536) (end 29.375 15.5743) (width 0.2) (layer "B.Cu") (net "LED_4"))
 (segment (start 27.9907 5.7875) (end 28.2516 6.0484) (width 0.2) (layer "B.Cu") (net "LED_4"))
 (segment (start 29.375 15.5743) (end 29.375 16.95) (width 0.2) (layer "B.Cu") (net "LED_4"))
 (segment (start 28.2516 6.0484) (end 29.8133 6.0484) (width 0.2) (layer "B.Cu") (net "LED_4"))
 (segment (start 30.1512 5.7105) (end 30.7917 5.7105) (width 0.2) (layer "B.Cu") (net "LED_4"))
 (segment (start 29.8133 6.0484) (end 30.1512 5.7105) (width 0.2) (layer "B.Cu") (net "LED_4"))
 (segment (start 30.7917 5.7105) (end 31.4133 6.3321) (width 0.2) (layer "B.Cu") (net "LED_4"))
 (segment (start 9 5.8244) (end 9 5.7875) (width 0.2) (layer "F.Cu") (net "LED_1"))
 (segment (start 9.7389 6.5633) (end 9 5.8244) (width 0.2) (layer "F.Cu") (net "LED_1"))
 (via (at 9.7389 6.5633) (size 0.6) (drill 0.3) (layers "F.Cu" "B.Cu") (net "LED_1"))
 (segment (start 12.336 3.9662) (end 9.7389 6.5633) (width 0.2) (layer "B.Cu") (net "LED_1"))
 (segment (start 30.7612 3.9662) (end 12.336 3.9662) (width 0.2) (layer "B.Cu") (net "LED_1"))
 (segment (start 33.125 16.95) (end 33.125 6.33) (width 0.2) (layer "B.Cu") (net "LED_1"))
 (segment (start 33.125 6.33) (end 30.7612 3.9662) (width 0.2) (layer "B.Cu") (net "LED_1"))
 (segment (start 33.9362 18.5214) (end 24.4356 18.5214) (width 0.2) (layer "B.Cu") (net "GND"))
 (segment (start 22.525 16.6108) (end 22.525 13.6) (width 0.2) (layer "B.Cu") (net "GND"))
 (segment (start 34.148 18.3096) (end 33.9362 18.5214) (width 0.2) (layer "B.Cu") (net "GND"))
 (segment (start 34.375 16.95) (end 34.375 16.7) (width 0.2) (layer "B.Cu") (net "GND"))
 (segment (start 34.375 16.95) (end 34.268 17.057) (width 0.2) (layer "B.Cu") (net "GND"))
 (segment (start 34.375 16.7) (end 37.475 13.6) (width 0.2) (layer "B.Cu") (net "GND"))
 (segment (start 34.268 18.3096) (end 34.148 18.3096) (width 0.15) (layer "B.Cu") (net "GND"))
 (segment (start 24.4356 18.5214) (end 22.525 16.6108) (width 0.2) (layer "B.Cu") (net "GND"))
 (segment (start 34.268 17.057) (end 34.268 18.3096) (width 0.2) (layer "B.Cu") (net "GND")))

